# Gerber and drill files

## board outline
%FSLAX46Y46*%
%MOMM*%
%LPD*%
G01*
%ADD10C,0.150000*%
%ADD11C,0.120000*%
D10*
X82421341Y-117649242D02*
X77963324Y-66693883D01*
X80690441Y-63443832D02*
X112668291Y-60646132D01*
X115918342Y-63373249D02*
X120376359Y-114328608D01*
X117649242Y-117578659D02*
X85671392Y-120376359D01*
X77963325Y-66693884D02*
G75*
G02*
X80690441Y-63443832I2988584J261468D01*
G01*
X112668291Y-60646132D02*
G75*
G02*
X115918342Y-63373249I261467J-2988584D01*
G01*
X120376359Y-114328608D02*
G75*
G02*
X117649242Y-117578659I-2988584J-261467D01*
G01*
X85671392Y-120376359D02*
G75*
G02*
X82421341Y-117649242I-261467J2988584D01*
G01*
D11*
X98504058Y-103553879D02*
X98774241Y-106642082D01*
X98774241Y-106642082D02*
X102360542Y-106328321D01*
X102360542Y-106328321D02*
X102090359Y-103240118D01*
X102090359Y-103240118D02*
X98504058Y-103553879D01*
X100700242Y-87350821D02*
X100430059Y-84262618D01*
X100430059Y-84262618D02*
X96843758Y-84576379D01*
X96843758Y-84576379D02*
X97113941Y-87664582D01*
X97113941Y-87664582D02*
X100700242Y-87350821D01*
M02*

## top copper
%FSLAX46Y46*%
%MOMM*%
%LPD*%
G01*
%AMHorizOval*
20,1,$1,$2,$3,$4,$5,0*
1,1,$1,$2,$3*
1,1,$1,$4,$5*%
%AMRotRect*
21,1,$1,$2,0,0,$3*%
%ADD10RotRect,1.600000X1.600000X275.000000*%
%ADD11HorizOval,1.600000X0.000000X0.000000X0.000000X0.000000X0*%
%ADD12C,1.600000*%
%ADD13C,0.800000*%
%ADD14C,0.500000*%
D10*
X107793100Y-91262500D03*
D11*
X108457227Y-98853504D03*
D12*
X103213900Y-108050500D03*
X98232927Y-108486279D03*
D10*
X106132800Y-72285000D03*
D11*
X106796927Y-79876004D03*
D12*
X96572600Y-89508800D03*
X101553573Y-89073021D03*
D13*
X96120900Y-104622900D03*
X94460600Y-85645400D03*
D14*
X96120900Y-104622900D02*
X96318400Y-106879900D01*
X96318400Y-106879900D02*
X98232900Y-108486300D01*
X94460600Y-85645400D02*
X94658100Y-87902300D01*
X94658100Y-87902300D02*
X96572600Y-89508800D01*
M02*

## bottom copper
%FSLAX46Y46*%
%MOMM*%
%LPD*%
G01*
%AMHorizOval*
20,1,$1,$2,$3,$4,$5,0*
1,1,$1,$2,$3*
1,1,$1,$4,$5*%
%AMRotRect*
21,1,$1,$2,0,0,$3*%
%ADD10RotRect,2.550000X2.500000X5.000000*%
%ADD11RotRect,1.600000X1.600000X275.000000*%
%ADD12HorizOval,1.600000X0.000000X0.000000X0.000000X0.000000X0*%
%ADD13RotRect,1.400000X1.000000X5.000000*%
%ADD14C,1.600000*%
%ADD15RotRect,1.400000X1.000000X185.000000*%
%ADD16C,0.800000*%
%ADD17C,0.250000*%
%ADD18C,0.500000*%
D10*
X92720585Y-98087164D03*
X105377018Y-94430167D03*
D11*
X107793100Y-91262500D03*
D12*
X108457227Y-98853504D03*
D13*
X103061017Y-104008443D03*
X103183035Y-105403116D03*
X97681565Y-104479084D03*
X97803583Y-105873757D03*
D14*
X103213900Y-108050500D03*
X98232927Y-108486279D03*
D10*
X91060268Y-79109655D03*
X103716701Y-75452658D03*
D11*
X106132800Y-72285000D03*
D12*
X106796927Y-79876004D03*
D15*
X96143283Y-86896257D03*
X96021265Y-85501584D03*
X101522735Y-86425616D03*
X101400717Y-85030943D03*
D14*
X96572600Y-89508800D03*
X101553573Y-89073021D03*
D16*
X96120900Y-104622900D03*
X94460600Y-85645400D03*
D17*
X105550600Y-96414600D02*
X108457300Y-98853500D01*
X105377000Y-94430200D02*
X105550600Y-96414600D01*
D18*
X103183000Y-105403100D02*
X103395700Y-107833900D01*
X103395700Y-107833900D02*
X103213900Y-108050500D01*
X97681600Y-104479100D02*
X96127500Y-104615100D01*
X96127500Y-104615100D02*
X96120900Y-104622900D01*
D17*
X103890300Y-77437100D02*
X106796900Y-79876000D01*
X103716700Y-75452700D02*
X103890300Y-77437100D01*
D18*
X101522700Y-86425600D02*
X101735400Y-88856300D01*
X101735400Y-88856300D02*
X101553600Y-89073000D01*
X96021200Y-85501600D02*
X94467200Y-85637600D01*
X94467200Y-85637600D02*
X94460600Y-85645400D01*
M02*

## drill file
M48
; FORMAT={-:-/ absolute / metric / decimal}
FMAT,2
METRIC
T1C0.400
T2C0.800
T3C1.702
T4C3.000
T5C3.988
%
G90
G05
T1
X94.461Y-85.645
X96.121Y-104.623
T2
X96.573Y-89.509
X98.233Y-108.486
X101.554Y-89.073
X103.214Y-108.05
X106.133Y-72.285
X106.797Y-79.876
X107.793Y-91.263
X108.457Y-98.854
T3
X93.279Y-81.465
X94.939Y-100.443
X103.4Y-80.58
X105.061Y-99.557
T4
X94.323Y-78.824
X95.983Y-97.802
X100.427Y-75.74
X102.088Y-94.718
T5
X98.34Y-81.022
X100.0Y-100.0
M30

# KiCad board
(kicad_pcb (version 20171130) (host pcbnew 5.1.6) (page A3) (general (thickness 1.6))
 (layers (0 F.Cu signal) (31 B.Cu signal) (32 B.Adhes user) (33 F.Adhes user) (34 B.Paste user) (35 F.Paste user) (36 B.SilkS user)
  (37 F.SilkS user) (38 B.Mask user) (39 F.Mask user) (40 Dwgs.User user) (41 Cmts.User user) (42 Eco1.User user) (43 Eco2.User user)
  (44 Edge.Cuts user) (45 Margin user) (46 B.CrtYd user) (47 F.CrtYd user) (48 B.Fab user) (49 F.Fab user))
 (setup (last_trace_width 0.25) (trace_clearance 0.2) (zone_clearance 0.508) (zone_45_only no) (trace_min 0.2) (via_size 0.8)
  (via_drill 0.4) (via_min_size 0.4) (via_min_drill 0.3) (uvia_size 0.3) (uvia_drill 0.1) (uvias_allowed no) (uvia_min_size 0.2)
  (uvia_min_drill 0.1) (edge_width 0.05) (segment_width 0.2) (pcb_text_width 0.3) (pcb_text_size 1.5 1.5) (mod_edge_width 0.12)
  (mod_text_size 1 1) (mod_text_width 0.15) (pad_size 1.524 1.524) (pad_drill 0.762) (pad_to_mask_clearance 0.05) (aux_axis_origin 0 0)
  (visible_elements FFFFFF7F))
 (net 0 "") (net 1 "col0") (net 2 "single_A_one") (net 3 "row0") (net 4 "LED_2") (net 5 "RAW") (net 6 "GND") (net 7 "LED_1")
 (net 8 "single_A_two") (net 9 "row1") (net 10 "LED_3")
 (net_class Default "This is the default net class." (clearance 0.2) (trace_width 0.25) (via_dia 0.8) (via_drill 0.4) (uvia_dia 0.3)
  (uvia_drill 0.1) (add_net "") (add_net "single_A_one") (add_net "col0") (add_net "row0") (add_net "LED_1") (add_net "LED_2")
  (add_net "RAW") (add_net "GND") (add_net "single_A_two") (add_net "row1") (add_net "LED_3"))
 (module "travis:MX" (layer F.Cu) (at 100 100 5)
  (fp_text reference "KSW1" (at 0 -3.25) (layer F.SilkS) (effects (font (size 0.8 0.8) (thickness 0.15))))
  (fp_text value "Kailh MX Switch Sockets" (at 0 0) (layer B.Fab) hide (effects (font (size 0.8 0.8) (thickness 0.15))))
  (pad "" np_thru_hole circle (at 0 0) (size 3.9878 3.9878) (drill 3.9878) (layers *.Cu *.Mask))
  (pad "" np_thru_hole circle (at 5.08 0) (size 1.7018 1.7018) (drill 1.7018) (layers *.Cu *.Mask))
  (pad "" np_thru_hole circle (at -5.08 0) (size 1.7018 1.7018) (drill 1.7018) (layers *.Cu *.Mask))
  (pad "" np_thru_hole circle (at 2.54 -5.08) (size 3 3) (drill 3) (layers *.Cu *.Mask))
  (pad "" np_thru_hole circle (at -3.81 -2.54) (size 3 3) (drill 3) (layers *.Cu *.Mask))
  (pad 1 smd rect (at -7.085 -2.54 5) (size 2.55 2.5) (layers B.Cu B.Paste B.Mask) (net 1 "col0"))
  (pad 2 smd rect (at 5.842 -5.08 5) (size 2.55 2.5) (layers B.Cu B.Paste B.Mask) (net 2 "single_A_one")))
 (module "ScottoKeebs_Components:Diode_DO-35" (layer "B.Cu") (at 107.7931 91.2625 275)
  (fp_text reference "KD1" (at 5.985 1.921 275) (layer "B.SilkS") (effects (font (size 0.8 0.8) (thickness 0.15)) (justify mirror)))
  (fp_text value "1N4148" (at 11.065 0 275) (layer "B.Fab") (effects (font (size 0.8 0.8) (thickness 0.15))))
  (pad 1 thru_hole rect (at 0 0 275) (size 1.6 1.6) (drill 0.8) (layers "*.Cu" "*.Mask") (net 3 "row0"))
  (pad 2 thru_hole oval (at 7.62 0 275) (size 1.6 1.6) (drill 0.8) (layers "*.Cu" "*.Mask") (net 2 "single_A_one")))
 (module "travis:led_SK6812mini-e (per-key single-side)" (layer B.Cu) (at 100.4323 104.9411 5)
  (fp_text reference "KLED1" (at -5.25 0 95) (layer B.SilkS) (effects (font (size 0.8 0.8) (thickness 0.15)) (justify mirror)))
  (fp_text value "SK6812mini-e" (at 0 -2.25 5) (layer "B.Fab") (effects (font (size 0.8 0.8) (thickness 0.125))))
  (pad 2 smd rect (at 2.70 -0.7 5) (size 1.4 1) (layers B.Cu B.Paste B.Mask) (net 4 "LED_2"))
  (pad 1 smd rect (at 2.70 0.7 5) (size 1.4 1) (layers B.Cu B.Paste B.Mask) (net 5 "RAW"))
  (pad 3 smd rect (at -2.70 -0.7 5) (size 1.4 1) (layers B.Cu B.Paste B.Mask) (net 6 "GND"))
  (pad 4 smd rect (at -2.70 0.7 5) (size 1.4 1) (layers B.Cu B.Paste B.Mask) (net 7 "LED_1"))
  (fp_line (start -1.8 -1.55) (end -1.8 1.55) (layer Edge.Cuts) (width 0.12))
  (fp_line (start -1.8 1.55) (end 1.8 1.55) (layer Edge.Cuts) (width 0.12))
  (fp_line (start 1.8 1.55) (end 1.8 -1.55) (layer Edge.Cuts) (width 0.12))
  (fp_line (start 1.8 -1.55) (end -1.8 -1.55) (layer Edge.Cuts) (width 0.12)))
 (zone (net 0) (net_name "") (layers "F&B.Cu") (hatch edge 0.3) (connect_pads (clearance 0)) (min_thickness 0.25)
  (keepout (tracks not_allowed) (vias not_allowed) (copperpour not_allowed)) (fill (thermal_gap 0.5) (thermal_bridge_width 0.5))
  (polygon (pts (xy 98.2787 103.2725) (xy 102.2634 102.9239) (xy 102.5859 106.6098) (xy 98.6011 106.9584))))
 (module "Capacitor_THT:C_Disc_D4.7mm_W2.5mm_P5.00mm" (layer B.Cu) (at 103.2139 108.0505 185)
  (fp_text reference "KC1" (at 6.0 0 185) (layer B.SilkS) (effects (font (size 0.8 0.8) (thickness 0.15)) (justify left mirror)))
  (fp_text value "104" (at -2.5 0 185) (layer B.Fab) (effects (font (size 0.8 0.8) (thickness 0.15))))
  (pad 1 thru_hole circle (at 0 0) (size 1.6 1.6) (drill 0.8) (layers *.Cu *.Mask) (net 5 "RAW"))
  (pad 2 thru_hole circle (at 5 0) (size 1.6 1.6) (drill 0.8) (layers *.Cu *.Mask) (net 6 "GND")))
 (segment (start 105.5506 96.4146) (end 108.4573 98.8535) (width 0.25) (layer "B.Cu") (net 2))
 (segment (start 105.3770 94.4302) (end 105.5506 96.4146) (width 0.25) (layer "B.Cu") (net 2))
 (segment (start 103.1830 105.4031) (end 103.3957 107.8339) (width 0.5) (layer "B.Cu") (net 5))
 (segment (start 103.3957 107.8339) (end 103.2139 108.0505) (width 0.5) (layer "B.Cu") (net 5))
 (segment (start 96.1209 104.6229) (end 96.3184 106.8799) (width 0.5) (layer "F.Cu") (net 6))
 (segment (start 96.3184 106.8799) (end 98.2329 108.4863) (width 0.5) (layer "F.Cu") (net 6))
 (via (at 96.1209 104.6229) (size 0.8) (drill 0.4) (layers "F.Cu" "B.Cu") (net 6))
 (segment (start 97.6816 104.4791) (end 96.1275 104.6151) (width 0.5) (layer "B.Cu") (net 6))
 (segment (start 96.1275 104.6151) (end 96.1209 104.6229) (width 0.5) (layer "B.Cu") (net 6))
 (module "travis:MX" (layer F.Cu) (at 98.3396831 81.022491 5)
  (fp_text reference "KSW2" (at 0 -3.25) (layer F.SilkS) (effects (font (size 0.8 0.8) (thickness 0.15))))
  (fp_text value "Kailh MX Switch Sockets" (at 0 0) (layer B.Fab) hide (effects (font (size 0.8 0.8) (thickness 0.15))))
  (pad "" np_thru_hole circle (at 0 0) (size 3.9878 3.9878) (drill 3.9878) (layers *.Cu *.Mask))
  (pad "" np_thru_hole circle (at 5.08 0) (size 1.7018 1.7018) (drill 1.7018) (layers *.Cu *.Mask))
  (pad "" np_thru_hole circle (at -5.08 0) (size 1.7018 1.7018) (drill 1.7018) (layers *.Cu *.Mask))
  (pad "" np_thru_hole circle (at 2.54 -5.08) (size 3 3) (drill 3) (layers *.Cu *.Mask))
  (pad "" np_thru_hole circle (at -3.81 -2.54) (size 3 3) (drill 3) (layers *.Cu *.Mask))
  (pad 1 smd rect (at -7.085 -2.54 5) (size 2.55 2.5) (layers B.Cu B.Paste B.Mask) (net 1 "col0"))
  (pad 2 smd rect (at 5.842 -5.08 5) (size 2.55 2.5) (layers B.Cu B.Paste B.Mask) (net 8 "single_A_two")))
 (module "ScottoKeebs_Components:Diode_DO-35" (layer "B.Cu") (at 106.1328 72.2850 275)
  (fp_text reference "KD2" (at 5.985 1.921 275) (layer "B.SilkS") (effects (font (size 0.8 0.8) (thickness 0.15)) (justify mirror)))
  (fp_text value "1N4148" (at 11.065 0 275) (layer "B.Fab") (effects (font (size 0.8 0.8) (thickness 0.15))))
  (pad 1 thru_hole rect (at 0 0 275) (size 1.6 1.6) (drill 0.8) (layers "*.Cu" "*.Mask") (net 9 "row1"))
  (pad 2 thru_hole oval (at 7.62 0 275) (size 1.6 1.6) (drill 0.8) (layers "*.Cu" "*.Mask") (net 8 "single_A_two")))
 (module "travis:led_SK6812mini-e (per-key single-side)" (layer B.Cu) (at 98.7720 85.9636 185)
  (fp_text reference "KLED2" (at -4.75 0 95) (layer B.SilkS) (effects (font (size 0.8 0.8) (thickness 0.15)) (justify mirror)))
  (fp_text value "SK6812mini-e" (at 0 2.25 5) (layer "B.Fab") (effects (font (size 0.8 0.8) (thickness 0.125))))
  (pad 2 smd rect (at 2.70 -0.7 185) (size 1.4 1) (layers B.Cu B.Paste B.Mask) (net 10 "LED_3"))
  (pad 1 smd rect (at 2.70 0.7 185) (size 1.4 1) (layers B.Cu B.Paste B.Mask) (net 5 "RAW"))
  (pad 3 smd rect (at -2.70 -0.7 185) (size 1.4 1) (layers B.Cu B.Paste B.Mask) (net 6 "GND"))
  (pad 4 smd rect (at -2.70 0.7 185) (size 1.4 1) (layers B.Cu B.Paste B.Mask) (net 4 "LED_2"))
  (fp_line (start -1.8 -1.55) (end -1.8 1.55) (layer Edge.Cuts) (width 0.12))
  (fp_line (start -1.8 1.55) (end 1.8 1.55) (layer Edge.Cuts) (width 0.12))
  (fp_line (start 1.8 1.55) (end 1.8 -1.55) (layer Edge.Cuts) (width 0.12))
  (fp_line (start 1.8 -1.55) (end -1.8 -1.55) (layer Edge.Cuts) (width 0.12)))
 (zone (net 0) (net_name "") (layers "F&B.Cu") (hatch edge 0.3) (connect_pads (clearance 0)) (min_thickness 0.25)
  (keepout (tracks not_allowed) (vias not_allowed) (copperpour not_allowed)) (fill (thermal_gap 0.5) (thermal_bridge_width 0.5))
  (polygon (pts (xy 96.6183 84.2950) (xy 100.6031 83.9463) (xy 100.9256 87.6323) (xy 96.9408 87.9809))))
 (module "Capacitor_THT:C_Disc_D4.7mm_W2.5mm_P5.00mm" (layer B.Cu) (at 96.5726 89.5088 5)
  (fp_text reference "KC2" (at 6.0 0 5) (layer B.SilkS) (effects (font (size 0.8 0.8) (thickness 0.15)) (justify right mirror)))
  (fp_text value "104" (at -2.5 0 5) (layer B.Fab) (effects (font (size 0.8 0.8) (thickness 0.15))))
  (pad 1 thru_hole circle (at 0 0) (size 1.6 1.6) (drill 0.8) (layers *.Cu *.Mask) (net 5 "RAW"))
  (pad 2 thru_hole circle (at 5 0) (size 1.6 1.6) (drill 0.8) (layers *.Cu *.Mask) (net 6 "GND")))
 (segment (start 103.8903 77.4371) (end 106.7969 79.8760) (width 0.25) (layer "B.Cu") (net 8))
 (segment (start 103.7167 75.4527) (end 103.8903 77.4371) (width 0.25) (layer "B.Cu") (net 8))
 (segment (start 101.5227 86.4256) (end 101.7354 88.8563) (width 0.5) (layer "B.Cu") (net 6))
 (segment (start 101.7354 88.8563) (end 101.5536 89.0730) (width 0.5) (layer "B.Cu") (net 6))
 (segment (start 94.4606 85.6454) (end 94.6581 87.9023) (width 0.5) (layer "F.Cu") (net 5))
 (segment (start 94.6581 87.9023) (end 96.5726 89.5088) (width 0.5) (layer "F.Cu") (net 5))
 (via (at 94.4606 85.6454) (size 0.8) (drill 0.4) (layers "F.Cu" "B.Cu") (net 5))
 (segment (start 96.0212 85.5016) (end 94.4672 85.6376) (width 0.5) (layer "B.Cu") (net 5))
 (segment (start 94.4672 85.6376) (end 94.4606 85.6454) (width 0.5) (layer "B.Cu") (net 5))
 (gr_line (start 82.42134066020488 117.64924167465301) (end 77.96332441742427 66.69388286964704) (angle 90) (layer Edge.Cuts) (width 0.15))
 (gr_line (start 80.69044142534706 63.44383166020488) (end 112.66829123035309 60.64613231742427) (angle 90) (layer Edge.Cuts) (width 0.15))
 (gr_line (start 115.91834243979514 63.37324932534716) (end 120.37635868257576 114.32860813035336) (angle 90) (layer Edge.Cuts) (width 0.15))
 (gr_line (start 117.64924167465291 117.57865933979514) (end 85.67139186964687 120.37635868257574) (angle 90) (layer Edge.Cuts) (width 0.15))
 (gr_arc (start 80.95190852610668 66.43241576888738) (end 80.69044142610667 63.443831668887384) (angle -90.00000000000101) (layer Edge.Cuts)
  (width 0.15))
 (gr_arc (start 112.9297583311127 63.63471642610668) (end 115.91834243111269 63.37324932610668) (angle -90.00000000000168) (layer Edge.Cuts)
  (width 0.15))
 (gr_arc (start 117.38777457389334 114.5900752311129) (end 117.64924167389334 117.5786593311129) (angle -89.99999999999918)
  (layer Edge.Cuts) (width 0.15))
 (gr_arc (start 85.40992476888728 117.38777457389334) (end 82.42134066888728 117.64924167389334) (angle -89.99999999999838)
  (layer Edge.Cuts) (width 0.15)))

